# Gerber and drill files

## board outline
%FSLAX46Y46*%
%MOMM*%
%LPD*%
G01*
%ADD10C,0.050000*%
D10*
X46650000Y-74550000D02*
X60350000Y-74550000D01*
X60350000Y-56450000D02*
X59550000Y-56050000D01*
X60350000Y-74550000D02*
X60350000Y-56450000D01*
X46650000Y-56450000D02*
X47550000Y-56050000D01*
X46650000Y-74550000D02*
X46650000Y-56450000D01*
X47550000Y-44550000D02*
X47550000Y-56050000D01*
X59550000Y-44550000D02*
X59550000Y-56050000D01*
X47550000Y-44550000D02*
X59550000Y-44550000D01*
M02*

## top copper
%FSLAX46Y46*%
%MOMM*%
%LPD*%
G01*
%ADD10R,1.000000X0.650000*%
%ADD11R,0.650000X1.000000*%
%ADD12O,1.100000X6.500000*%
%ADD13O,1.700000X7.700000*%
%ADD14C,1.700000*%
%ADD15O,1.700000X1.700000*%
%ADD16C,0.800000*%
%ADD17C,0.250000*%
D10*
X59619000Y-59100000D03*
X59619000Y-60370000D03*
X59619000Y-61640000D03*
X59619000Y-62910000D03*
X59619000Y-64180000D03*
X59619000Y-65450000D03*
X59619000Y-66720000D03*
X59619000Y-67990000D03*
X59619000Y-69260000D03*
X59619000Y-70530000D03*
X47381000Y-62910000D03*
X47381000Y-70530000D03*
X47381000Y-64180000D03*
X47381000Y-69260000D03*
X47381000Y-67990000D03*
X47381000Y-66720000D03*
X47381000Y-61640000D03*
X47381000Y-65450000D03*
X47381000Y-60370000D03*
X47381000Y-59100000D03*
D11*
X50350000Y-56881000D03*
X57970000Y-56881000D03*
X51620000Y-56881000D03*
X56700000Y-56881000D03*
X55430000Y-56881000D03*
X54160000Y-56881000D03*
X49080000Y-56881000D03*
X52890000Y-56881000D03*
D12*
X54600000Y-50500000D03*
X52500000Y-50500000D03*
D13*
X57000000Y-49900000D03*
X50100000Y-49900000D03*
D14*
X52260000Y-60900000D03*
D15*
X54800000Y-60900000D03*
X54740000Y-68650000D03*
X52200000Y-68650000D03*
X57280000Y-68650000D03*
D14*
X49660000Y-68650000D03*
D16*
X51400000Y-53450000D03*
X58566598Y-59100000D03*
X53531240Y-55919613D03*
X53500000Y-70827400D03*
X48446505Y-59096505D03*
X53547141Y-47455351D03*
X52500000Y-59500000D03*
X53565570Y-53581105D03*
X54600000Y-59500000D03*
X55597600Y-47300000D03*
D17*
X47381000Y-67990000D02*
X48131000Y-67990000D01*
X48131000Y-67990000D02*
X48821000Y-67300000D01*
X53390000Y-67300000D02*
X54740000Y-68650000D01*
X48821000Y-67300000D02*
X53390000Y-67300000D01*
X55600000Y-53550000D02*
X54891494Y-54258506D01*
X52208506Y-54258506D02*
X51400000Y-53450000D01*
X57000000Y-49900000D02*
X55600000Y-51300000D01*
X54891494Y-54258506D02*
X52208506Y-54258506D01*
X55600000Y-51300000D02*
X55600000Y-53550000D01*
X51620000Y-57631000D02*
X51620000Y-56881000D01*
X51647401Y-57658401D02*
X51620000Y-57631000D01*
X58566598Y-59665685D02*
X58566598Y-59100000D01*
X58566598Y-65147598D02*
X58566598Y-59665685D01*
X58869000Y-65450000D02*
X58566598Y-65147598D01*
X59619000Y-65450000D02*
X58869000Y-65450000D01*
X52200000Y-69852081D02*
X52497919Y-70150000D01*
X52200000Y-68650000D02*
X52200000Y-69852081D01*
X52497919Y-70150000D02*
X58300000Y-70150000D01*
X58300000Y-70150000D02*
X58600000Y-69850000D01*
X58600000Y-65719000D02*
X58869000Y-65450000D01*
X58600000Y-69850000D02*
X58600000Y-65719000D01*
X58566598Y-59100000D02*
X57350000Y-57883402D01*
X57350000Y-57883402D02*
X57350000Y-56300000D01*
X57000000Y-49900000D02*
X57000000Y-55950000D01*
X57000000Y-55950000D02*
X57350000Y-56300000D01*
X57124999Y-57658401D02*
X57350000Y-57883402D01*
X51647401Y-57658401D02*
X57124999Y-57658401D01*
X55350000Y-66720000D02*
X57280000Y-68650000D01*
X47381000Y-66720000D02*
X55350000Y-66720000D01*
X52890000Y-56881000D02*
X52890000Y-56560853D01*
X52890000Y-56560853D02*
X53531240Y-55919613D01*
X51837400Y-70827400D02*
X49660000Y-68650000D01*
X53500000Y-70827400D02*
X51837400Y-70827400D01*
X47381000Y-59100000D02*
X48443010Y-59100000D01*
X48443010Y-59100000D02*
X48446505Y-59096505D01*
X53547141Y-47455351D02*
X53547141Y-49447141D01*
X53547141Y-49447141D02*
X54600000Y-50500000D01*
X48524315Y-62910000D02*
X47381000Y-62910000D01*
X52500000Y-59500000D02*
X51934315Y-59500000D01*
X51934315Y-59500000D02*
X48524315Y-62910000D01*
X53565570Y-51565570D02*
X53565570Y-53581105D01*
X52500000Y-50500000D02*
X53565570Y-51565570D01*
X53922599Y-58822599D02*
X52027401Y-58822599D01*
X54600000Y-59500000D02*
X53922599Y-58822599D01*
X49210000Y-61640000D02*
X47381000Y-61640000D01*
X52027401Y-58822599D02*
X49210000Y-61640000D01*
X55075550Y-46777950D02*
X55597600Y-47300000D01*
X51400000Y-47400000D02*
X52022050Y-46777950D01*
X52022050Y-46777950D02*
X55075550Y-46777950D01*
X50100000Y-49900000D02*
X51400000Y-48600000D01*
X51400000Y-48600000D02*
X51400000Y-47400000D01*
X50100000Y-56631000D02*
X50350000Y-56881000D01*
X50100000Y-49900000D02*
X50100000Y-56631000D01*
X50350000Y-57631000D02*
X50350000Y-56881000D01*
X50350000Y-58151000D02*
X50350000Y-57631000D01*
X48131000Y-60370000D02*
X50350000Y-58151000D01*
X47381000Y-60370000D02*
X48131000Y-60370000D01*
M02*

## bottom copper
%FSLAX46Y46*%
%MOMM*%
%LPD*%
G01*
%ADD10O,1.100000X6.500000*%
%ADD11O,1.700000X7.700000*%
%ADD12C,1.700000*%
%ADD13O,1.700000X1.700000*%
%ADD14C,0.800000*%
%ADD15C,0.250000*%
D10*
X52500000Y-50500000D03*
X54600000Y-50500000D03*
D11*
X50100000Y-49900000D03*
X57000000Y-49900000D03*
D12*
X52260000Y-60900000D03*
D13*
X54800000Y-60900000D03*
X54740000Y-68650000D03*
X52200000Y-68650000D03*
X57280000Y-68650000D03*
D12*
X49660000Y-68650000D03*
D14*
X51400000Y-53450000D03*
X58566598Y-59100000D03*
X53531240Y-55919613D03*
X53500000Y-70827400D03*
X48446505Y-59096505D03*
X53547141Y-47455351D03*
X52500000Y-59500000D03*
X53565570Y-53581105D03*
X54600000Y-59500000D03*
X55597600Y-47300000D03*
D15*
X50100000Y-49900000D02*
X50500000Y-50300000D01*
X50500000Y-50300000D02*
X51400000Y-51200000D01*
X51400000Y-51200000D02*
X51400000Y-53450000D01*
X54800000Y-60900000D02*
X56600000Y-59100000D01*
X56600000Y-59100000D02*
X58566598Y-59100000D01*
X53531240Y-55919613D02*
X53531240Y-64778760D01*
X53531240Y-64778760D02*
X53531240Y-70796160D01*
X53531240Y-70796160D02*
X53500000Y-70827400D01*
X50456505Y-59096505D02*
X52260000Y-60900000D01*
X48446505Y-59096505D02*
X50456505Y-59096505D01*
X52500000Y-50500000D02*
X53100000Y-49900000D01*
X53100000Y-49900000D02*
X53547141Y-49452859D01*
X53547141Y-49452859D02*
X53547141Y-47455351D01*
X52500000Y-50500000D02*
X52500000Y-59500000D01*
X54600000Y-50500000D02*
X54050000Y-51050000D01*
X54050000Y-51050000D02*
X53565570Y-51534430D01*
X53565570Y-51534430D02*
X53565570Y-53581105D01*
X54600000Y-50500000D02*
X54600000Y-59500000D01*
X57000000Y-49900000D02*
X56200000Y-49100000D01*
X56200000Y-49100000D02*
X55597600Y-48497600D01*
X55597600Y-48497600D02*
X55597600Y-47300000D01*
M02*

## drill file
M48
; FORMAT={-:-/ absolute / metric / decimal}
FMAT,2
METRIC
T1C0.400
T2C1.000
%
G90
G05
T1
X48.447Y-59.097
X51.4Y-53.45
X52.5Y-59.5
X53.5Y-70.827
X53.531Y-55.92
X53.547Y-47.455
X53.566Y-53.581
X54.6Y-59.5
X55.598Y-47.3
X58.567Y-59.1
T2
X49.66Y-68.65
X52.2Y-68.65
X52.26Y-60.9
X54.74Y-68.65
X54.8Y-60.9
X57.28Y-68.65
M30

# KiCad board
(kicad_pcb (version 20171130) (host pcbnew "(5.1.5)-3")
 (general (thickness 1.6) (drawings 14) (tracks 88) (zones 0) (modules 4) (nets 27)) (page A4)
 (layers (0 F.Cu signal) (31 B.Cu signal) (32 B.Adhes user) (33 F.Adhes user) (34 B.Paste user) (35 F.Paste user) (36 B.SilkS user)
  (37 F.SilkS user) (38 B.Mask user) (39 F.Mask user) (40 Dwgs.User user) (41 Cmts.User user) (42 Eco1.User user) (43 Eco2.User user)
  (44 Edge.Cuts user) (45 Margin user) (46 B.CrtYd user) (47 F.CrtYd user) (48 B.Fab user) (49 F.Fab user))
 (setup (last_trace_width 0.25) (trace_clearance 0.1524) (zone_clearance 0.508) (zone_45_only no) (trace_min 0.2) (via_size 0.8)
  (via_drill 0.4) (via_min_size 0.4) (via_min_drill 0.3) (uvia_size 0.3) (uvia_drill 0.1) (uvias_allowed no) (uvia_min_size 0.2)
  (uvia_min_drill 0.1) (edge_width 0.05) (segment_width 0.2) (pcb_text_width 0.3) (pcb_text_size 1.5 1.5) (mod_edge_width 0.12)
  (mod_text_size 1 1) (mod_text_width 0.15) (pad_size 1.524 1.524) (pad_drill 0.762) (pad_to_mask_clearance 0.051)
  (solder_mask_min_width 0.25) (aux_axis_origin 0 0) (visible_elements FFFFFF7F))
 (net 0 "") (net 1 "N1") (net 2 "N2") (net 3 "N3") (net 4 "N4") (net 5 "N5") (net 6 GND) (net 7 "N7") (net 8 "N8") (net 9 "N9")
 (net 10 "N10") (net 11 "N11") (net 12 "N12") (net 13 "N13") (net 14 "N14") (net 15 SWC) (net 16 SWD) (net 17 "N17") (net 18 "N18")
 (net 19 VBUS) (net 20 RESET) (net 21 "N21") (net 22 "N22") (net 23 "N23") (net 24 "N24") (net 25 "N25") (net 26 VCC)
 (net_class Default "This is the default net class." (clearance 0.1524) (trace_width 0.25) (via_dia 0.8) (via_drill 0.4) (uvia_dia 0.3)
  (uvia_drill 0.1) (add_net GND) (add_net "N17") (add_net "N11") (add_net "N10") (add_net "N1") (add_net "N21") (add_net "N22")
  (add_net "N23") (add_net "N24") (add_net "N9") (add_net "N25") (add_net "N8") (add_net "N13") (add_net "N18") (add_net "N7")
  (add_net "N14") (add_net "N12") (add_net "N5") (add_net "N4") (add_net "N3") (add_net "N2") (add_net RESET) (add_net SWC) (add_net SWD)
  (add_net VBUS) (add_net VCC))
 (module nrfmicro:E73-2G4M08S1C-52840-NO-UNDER (layer F.Cu) (at 53.5 56.5 270)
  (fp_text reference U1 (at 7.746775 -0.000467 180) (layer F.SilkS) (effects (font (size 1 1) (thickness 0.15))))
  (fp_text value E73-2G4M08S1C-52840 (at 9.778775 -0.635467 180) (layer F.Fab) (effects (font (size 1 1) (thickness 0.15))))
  (pad 10 smd rect (at 2.6 -6.119 270) (size 0.65 1) (layers F.Cu F.Paste F.Mask) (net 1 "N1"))
  (pad 9 smd rect (at 3.87 -6.119 270) (size 0.65 1) (layers F.Cu F.Paste F.Mask) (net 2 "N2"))
  (pad 8 smd rect (at 5.14 -6.119 270) (size 0.65 1) (layers F.Cu F.Paste F.Mask) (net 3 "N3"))
  (pad 7 smd rect (at 6.41 -6.119 270) (size 0.65 1) (layers F.Cu F.Paste F.Mask) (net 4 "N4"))
  (pad 6 smd rect (at 7.68 -6.119 270) (size 0.65 1) (layers F.Cu F.Paste F.Mask) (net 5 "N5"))
  (pad 5 smd rect (at 8.95 -6.119 270) (size 0.65 1) (layers F.Cu F.Paste F.Mask) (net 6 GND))
  (pad 4 smd rect (at 10.22 -6.119 270) (size 0.65 1) (layers F.Cu F.Paste F.Mask) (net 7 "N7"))
  (pad 3 smd rect (at 11.49 -6.119 270) (size 0.65 1) (layers F.Cu F.Paste F.Mask) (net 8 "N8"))
  (pad 2 smd rect (at 12.76 -6.119 270) (size 0.65 1) (layers F.Cu F.Paste F.Mask) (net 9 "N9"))
  (pad 1 smd rect (at 14.03 -6.119 270) (size 0.65 1) (layers F.Cu F.Paste F.Mask) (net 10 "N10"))
  (pad 31 smd rect (at 6.41 6.119 270) (size 0.65 1) (layers F.Cu F.Paste F.Mask) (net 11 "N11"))
  (pad 43 smd rect (at 14.03 6.119 270) (size 0.65 1) (layers F.Cu F.Paste F.Mask) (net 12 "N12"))
  (pad 33 smd rect (at 7.68 6.119 270) (size 0.65 1) (layers F.Cu F.Paste F.Mask) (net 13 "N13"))
  (pad 41 smd rect (at 12.76 6.119 270) (size 0.65 1) (layers F.Cu F.Paste F.Mask) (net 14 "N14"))
  (pad 39 smd rect (at 11.49 6.119 270) (size 0.65 1) (layers F.Cu F.Paste F.Mask) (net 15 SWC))
  (pad 37 smd rect (at 10.22 6.119 270) (size 0.65 1) (layers F.Cu F.Paste F.Mask) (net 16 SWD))
  (pad 29 smd rect (at 5.14 6.119 270) (size 0.65 1) (layers F.Cu F.Paste F.Mask) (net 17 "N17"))
  (pad 35 smd rect (at 8.95 6.119 270) (size 0.65 1) (layers F.Cu F.Paste F.Mask) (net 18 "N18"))
  (pad 27 smd rect (at 3.87 6.119 270) (size 0.65 1) (layers F.Cu F.Paste F.Mask) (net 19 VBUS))
  (pad 26 smd rect (at 2.6 6.119 270) (size 0.65 1) (layers F.Cu F.Paste F.Mask) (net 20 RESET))
  (pad 23 smd rect (at 0.381 3.15) (size 0.65 1) (layers F.Cu F.Paste F.Mask) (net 19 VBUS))
  (pad 11 smd rect (at 0.381 -4.47) (size 0.65 1) (layers F.Cu F.Paste F.Mask) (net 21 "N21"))
  (pad 21 smd rect (at 0.381 1.88) (size 0.65 1) (layers F.Cu F.Paste F.Mask) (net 6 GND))
  (pad 13 smd rect (at 0.381 -3.2) (size 0.65 1) (layers F.Cu F.Paste F.Mask) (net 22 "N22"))
  (pad 15 smd rect (at 0.381 -1.93) (size 0.65 1) (layers F.Cu F.Paste F.Mask) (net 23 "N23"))
  (pad 17 smd rect (at 0.381 -0.66) (size 0.65 1) (layers F.Cu F.Paste F.Mask) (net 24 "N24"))
  (pad 25 smd rect (at 0.381 4.42) (size 0.65 1) (layers F.Cu F.Paste F.Mask) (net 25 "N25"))
  (pad 19 smd rect (at 0.381 0.61) (size 0.65 1) (layers F.Cu F.Paste F.Mask) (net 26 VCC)))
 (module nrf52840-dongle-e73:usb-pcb (layer F.Cu) (at 53.55 49.9)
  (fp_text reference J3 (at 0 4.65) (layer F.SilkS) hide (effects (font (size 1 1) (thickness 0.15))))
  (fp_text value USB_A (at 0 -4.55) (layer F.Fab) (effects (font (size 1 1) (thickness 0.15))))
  (pad 3 smd oval (at -1.05 0.6) (size 1.1 6.5) (layers B.Cu B.Paste B.Mask) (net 11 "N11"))
  (pad 2 smd oval (at 1.05 0.6) (size 1.1 6.5) (layers B.Cu B.Paste B.Mask) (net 17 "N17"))
  (pad 4 smd oval (at -3.45 0) (size 1.7 7.7) (layers B.Cu B.Paste B.Mask) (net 6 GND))
  (pad 1 smd oval (at 3.45 0) (size 1.7 7.7) (layers B.Cu B.Paste B.Mask) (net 19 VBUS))
  (pad 3 smd oval (at 1.05 0.6) (size 1.1 6.5) (layers F.Cu F.Paste F.Mask) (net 11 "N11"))
  (pad 2 smd oval (at -1.05 0.6) (size 1.1 6.5) (layers F.Cu F.Paste F.Mask) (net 17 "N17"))
  (pad 4 smd oval (at 3.45 0) (size 1.7 7.7) (layers F.Cu F.Paste F.Mask) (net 6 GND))
  (pad 1 smd oval (at -3.45 0) (size 1.7 7.7) (layers F.Cu F.Paste F.Mask) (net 19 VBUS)))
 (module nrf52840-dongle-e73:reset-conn (layer F.Cu) (at 52.26 60.9 90)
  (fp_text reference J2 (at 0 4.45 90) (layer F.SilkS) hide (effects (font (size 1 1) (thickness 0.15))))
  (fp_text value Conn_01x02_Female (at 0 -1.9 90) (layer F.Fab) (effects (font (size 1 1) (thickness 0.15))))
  (pad 1 thru_hole circle (at 0 0 90) (size 1.7 1.7) (drill 1) (layers *.Cu *.Mask) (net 20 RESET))
  (pad 2 thru_hole oval (at 0 2.54 90) (size 1.7 1.7) (drill 1) (layers *.Cu *.Mask) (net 6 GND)))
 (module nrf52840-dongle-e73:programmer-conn (layer B.Cu) (at 49.66 68.65 270)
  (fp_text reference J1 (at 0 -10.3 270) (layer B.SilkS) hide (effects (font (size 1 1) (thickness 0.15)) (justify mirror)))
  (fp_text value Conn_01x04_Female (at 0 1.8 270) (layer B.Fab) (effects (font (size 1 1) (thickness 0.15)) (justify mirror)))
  (pad 3 thru_hole oval (at 0 -5.08 270) (size 1.7 1.7) (drill 1) (layers *.Cu *.Mask) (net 15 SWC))
  (pad 2 thru_hole oval (at 0 -2.54 270) (size 1.7 1.7) (drill 1) (layers *.Cu *.Mask) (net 6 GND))
  (pad 4 thru_hole oval (at 0 -7.62 270) (size 1.7 1.7) (drill 1) (layers *.Cu *.Mask) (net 16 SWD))
  (pad 1 thru_hole circle (at 0 0 270) (size 1.7 1.7) (drill 1) (layers *.Cu *.Mask) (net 26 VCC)))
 (gr_line (start 46.65 74.55) (end 60.35 74.55) (layer Edge.Cuts) (width 0.05))
 (gr_line (start 60.35 56.45) (end 59.55 56.05) (layer Edge.Cuts) (width 0.05))
 (gr_line (start 60.35 74.55) (end 60.35 56.45) (layer Edge.Cuts) (width 0.05))
 (gr_line (start 46.65 56.45) (end 47.55 56.05) (layer Edge.Cuts) (width 0.05))
 (gr_line (start 46.65 74.55) (end 46.65 56.45) (layer Edge.Cuts) (width 0.05))
 (gr_line (start 47.55 44.55) (end 47.55 56.05) (layer Edge.Cuts) (width 0.05))
 (gr_line (start 59.55 44.55) (end 59.55 56.05) (layer Edge.Cuts) (width 0.05))
 (gr_line (start 47.55 44.55) (end 59.55 44.55) (layer Edge.Cuts) (width 0.05))
 (segment (start 47.381 67.99) (end 48.131 67.99) (width 0.25) (layer F.Cu) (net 15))
 (segment (start 48.131 67.99) (end 48.821 67.3) (width 0.25) (layer F.Cu) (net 15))
 (segment (start 53.39 67.3) (end 54.74 68.65) (width 0.25) (layer F.Cu) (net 15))
 (segment (start 48.821 67.3) (end 53.39 67.3) (width 0.25) (layer F.Cu) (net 15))
 (segment (start 50.1 49.9) (end 50.5 50.3) (width 0.25) (layer B.Cu) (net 6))
 (via (at 51.4 53.45) (size 0.8) (drill 0.4) (layers F.Cu B.Cu) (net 6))
 (segment (start 50.5 50.3) (end 51.4 51.2) (width 0.25) (layer B.Cu) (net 6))
 (segment (start 51.4 51.2) (end 51.4 53.45) (width 0.25) (layer B.Cu) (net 6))
 (segment (start 55.6 53.55) (end 54.891494 54.258506) (width 0.25) (layer F.Cu) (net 6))
 (segment (start 52.208506 54.258506) (end 51.4 53.45) (width 0.25) (layer F.Cu) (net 6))
 (segment (start 57 49.9) (end 55.6 51.3) (width 0.25) (layer F.Cu) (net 6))
 (segment (start 54.891494 54.258506) (end 52.208506 54.258506) (width 0.25) (layer F.Cu) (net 6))
 (segment (start 55.6 51.3) (end 55.6 53.55) (width 0.25) (layer F.Cu) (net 6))
 (segment (start 51.62 57.631) (end 51.62 56.881) (width 0.25) (layer F.Cu) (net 6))
 (segment (start 51.647401 57.658401) (end 51.62 57.631) (width 0.25) (layer F.Cu) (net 6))
 (segment (start 54.8 60.9) (end 56.6 59.1) (width 0.25) (layer B.Cu) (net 6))
 (via (at 58.566598 59.1) (size 0.8) (drill 0.4) (layers F.Cu B.Cu) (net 6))
 (segment (start 56.6 59.1) (end 58.566598 59.1) (width 0.25) (layer B.Cu) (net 6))
 (segment (start 58.566598 59.665685) (end 58.566598 59.1) (width 0.25) (layer F.Cu) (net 6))
 (segment (start 58.566598 65.147598) (end 58.566598 59.665685) (width 0.25) (layer F.Cu) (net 6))
 (segment (start 58.869 65.45) (end 58.566598 65.147598) (width 0.25) (layer F.Cu) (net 6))
 (segment (start 59.619 65.45) (end 58.869 65.45) (width 0.25) (layer F.Cu) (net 6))
 (segment (start 52.2 69.852081) (end 52.497919 70.15) (width 0.25) (layer F.Cu) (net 6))
 (segment (start 52.2 68.65) (end 52.2 69.852081) (width 0.25) (layer F.Cu) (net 6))
 (segment (start 52.497919 70.15) (end 58.3 70.15) (width 0.25) (layer F.Cu) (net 6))
 (segment (start 58.3 70.15) (end 58.6 69.85) (width 0.25) (layer F.Cu) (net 6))
 (segment (start 58.6 65.719) (end 58.869 65.45) (width 0.25) (layer F.Cu) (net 6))
 (segment (start 58.6 69.85) (end 58.6 65.719) (width 0.25) (layer F.Cu) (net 6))
 (segment (start 58.566598 59.1) (end 57.35 57.883402) (width 0.25) (layer F.Cu) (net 6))
 (segment (start 57.35 57.883402) (end 57.35 56.3) (width 0.25) (layer F.Cu) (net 6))
 (segment (start 57 49.9) (end 57 55.95) (width 0.25) (layer F.Cu) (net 6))
 (segment (start 57 55.95) (end 57.35 56.3) (width 0.25) (layer F.Cu) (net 6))
 (segment (start 57.124999 57.658401) (end 57.35 57.883402) (width 0.25) (layer F.Cu) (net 6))
 (segment (start 51.647401 57.658401) (end 57.124999 57.658401) (width 0.25) (layer F.Cu) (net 6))
 (segment (start 55.35 66.72) (end 57.28 68.65) (width 0.25) (layer F.Cu) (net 16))
 (segment (start 47.381 66.72) (end 55.35 66.72) (width 0.25) (layer F.Cu) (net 16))
 (via (at 53.53124 55.919613) (size 0.8) (drill 0.4) (layers F.Cu B.Cu) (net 26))
 (segment (start 52.89 56.881) (end 52.89 56.560853) (width 0.25) (layer F.Cu) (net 26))
 (segment (start 52.89 56.560853) (end 53.53124 55.919613) (width 0.25) (layer F.Cu) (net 26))
 (segment (start 53.53124 55.919613) (end 53.53124 64.77876) (width 0.25) (layer B.Cu) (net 26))
 (via (at 53.5 70.8274) (size 0.8) (drill 0.4) (layers F.Cu B.Cu) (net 26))
 (segment (start 53.53124 64.77876) (end 53.53124 70.79616) (width 0.25) (layer B.Cu) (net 26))
 (segment (start 53.53124 70.79616) (end 53.5 70.8274) (width 0.25) (layer B.Cu) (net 26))
 (segment (start 51.8374 70.8274) (end 49.66 68.65) (width 0.25) (layer F.Cu) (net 26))
 (segment (start 53.5 70.8274) (end 51.8374 70.8274) (width 0.25) (layer F.Cu) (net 26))
 (segment (start 47.381 59.1) (end 48.44301 59.1) (width 0.25) (layer F.Cu) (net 20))
 (via (at 48.446505 59.096505) (size 0.8) (drill 0.4) (layers F.Cu B.Cu) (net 20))
 (segment (start 48.44301 59.1) (end 48.446505 59.096505) (width 0.25) (layer F.Cu) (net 20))
 (segment (start 50.456505 59.096505) (end 52.26 60.9) (width 0.25) (layer B.Cu) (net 20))
 (segment (start 48.446505 59.096505) (end 50.456505 59.096505) (width 0.25) (layer B.Cu) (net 20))
 (segment (start 52.5 50.5) (end 53.1 49.9) (width 0.25) (layer B.Cu) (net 11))
 (via (at 53.547141 47.455351) (size 0.8) (drill 0.4) (layers F.Cu B.Cu) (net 11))
 (segment (start 53.1 49.9) (end 53.547141 49.452859) (width 0.25) (layer B.Cu) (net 11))
 (segment (start 53.547141 49.452859) (end 53.547141 47.455351) (width 0.25) (layer B.Cu) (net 11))
 (segment (start 53.547141 47.455351) (end 53.547141 49.447141) (width 0.25) (layer F.Cu) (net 11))
 (segment (start 53.547141 49.447141) (end 54.6 50.5) (width 0.25) (layer F.Cu) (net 11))
 (via (at 52.5 59.5) (size 0.8) (drill 0.4) (layers F.Cu B.Cu) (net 11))
 (segment (start 52.5 50.5) (end 52.5 59.5) (width 0.25) (layer B.Cu) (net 11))
 (segment (start 48.524315 62.91) (end 47.381 62.91) (width 0.25) (layer F.Cu) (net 11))
 (segment (start 52.5 59.5) (end 51.934315 59.5) (width 0.25) (layer F.Cu) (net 11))
 (segment (start 51.934315 59.5) (end 48.524315 62.91) (width 0.25) (layer F.Cu) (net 11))
 (segment (start 54.6 50.5) (end 54.05 51.05) (width 0.25) (layer B.Cu) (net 17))
 (segment (start 54.05 51.05) (end 53.56557 51.53443) (width 0.25) (layer B.Cu) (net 17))
 (via (at 53.56557 53.581105) (size 0.8) (drill 0.4) (layers F.Cu B.Cu) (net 17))
 (segment (start 53.56557 51.53443) (end 53.56557 53.581105) (width 0.25) (layer B.Cu) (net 17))
 (segment (start 53.56557 51.56557) (end 53.56557 53.581105) (width 0.25) (layer F.Cu) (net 17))
 (segment (start 52.5 50.5) (end 53.56557 51.56557) (width 0.25) (layer F.Cu) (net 17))
 (via (at 54.6 59.5) (size 0.8) (drill 0.4) (layers F.Cu B.Cu) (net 17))
 (segment (start 54.6 50.5) (end 54.6 59.5) (width 0.25) (layer B.Cu) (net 17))
 (segment (start 53.922599 58.822599) (end 52.027401 58.822599) (width 0.25) (layer F.Cu) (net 17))
 (segment (start 54.6 59.5) (end 53.922599 58.822599) (width 0.25) (layer F.Cu) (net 17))
 (segment (start 49.21 61.64) (end 47.381 61.64) (width 0.25) (layer F.Cu) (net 17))
 (segment (start 52.027401 58.822599) (end 49.21 61.64) (width 0.25) (layer F.Cu) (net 17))
 (segment (start 57 49.9) (end 56.2 49.1) (width 0.25) (layer B.Cu) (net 19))
 (via (at 55.5976 47.3) (size 0.8) (drill 0.4) (layers F.Cu B.Cu) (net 19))
 (segment (start 56.2 49.1) (end 55.5976 48.4976) (width 0.25) (layer B.Cu) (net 19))
 (segment (start 55.5976 48.4976) (end 55.5976 47.3) (width 0.25) (layer B.Cu) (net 19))
 (segment (start 55.07555 46.77795) (end 55.5976 47.3) (width 0.25) (layer F.Cu) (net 19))
 (segment (start 51.4 47.4) (end 52.02205 46.77795) (width 0.25) (layer F.Cu) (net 19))
 (segment (start 52.02205 46.77795) (end 55.07555 46.77795) (width 0.25) (layer F.Cu) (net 19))
 (segment (start 50.1 49.9) (end 51.4 48.6) (width 0.25) (layer F.Cu) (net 19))
 (segment (start 51.4 48.6) (end 51.4 47.4) (width 0.25) (layer F.Cu) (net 19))
 (segment (start 50.1 56.631) (end 50.35 56.881) (width 0.25) (layer F.Cu) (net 19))
 (segment (start 50.1 49.9) (end 50.1 56.631) (width 0.25) (layer F.Cu) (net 19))
 (segment (start 50.35 57.631) (end 50.35 56.881) (width 0.25) (layer F.Cu) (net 19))
 (segment (start 50.35 58.151) (end 50.35 57.631) (width 0.25) (layer F.Cu) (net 19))
 (segment (start 48.131 60.37) (end 50.35 58.151) (width 0.25) (layer F.Cu) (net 19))
 (segment (start 47.381 60.37) (end 48.131 60.37) (width 0.25) (layer F.Cu) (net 19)))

